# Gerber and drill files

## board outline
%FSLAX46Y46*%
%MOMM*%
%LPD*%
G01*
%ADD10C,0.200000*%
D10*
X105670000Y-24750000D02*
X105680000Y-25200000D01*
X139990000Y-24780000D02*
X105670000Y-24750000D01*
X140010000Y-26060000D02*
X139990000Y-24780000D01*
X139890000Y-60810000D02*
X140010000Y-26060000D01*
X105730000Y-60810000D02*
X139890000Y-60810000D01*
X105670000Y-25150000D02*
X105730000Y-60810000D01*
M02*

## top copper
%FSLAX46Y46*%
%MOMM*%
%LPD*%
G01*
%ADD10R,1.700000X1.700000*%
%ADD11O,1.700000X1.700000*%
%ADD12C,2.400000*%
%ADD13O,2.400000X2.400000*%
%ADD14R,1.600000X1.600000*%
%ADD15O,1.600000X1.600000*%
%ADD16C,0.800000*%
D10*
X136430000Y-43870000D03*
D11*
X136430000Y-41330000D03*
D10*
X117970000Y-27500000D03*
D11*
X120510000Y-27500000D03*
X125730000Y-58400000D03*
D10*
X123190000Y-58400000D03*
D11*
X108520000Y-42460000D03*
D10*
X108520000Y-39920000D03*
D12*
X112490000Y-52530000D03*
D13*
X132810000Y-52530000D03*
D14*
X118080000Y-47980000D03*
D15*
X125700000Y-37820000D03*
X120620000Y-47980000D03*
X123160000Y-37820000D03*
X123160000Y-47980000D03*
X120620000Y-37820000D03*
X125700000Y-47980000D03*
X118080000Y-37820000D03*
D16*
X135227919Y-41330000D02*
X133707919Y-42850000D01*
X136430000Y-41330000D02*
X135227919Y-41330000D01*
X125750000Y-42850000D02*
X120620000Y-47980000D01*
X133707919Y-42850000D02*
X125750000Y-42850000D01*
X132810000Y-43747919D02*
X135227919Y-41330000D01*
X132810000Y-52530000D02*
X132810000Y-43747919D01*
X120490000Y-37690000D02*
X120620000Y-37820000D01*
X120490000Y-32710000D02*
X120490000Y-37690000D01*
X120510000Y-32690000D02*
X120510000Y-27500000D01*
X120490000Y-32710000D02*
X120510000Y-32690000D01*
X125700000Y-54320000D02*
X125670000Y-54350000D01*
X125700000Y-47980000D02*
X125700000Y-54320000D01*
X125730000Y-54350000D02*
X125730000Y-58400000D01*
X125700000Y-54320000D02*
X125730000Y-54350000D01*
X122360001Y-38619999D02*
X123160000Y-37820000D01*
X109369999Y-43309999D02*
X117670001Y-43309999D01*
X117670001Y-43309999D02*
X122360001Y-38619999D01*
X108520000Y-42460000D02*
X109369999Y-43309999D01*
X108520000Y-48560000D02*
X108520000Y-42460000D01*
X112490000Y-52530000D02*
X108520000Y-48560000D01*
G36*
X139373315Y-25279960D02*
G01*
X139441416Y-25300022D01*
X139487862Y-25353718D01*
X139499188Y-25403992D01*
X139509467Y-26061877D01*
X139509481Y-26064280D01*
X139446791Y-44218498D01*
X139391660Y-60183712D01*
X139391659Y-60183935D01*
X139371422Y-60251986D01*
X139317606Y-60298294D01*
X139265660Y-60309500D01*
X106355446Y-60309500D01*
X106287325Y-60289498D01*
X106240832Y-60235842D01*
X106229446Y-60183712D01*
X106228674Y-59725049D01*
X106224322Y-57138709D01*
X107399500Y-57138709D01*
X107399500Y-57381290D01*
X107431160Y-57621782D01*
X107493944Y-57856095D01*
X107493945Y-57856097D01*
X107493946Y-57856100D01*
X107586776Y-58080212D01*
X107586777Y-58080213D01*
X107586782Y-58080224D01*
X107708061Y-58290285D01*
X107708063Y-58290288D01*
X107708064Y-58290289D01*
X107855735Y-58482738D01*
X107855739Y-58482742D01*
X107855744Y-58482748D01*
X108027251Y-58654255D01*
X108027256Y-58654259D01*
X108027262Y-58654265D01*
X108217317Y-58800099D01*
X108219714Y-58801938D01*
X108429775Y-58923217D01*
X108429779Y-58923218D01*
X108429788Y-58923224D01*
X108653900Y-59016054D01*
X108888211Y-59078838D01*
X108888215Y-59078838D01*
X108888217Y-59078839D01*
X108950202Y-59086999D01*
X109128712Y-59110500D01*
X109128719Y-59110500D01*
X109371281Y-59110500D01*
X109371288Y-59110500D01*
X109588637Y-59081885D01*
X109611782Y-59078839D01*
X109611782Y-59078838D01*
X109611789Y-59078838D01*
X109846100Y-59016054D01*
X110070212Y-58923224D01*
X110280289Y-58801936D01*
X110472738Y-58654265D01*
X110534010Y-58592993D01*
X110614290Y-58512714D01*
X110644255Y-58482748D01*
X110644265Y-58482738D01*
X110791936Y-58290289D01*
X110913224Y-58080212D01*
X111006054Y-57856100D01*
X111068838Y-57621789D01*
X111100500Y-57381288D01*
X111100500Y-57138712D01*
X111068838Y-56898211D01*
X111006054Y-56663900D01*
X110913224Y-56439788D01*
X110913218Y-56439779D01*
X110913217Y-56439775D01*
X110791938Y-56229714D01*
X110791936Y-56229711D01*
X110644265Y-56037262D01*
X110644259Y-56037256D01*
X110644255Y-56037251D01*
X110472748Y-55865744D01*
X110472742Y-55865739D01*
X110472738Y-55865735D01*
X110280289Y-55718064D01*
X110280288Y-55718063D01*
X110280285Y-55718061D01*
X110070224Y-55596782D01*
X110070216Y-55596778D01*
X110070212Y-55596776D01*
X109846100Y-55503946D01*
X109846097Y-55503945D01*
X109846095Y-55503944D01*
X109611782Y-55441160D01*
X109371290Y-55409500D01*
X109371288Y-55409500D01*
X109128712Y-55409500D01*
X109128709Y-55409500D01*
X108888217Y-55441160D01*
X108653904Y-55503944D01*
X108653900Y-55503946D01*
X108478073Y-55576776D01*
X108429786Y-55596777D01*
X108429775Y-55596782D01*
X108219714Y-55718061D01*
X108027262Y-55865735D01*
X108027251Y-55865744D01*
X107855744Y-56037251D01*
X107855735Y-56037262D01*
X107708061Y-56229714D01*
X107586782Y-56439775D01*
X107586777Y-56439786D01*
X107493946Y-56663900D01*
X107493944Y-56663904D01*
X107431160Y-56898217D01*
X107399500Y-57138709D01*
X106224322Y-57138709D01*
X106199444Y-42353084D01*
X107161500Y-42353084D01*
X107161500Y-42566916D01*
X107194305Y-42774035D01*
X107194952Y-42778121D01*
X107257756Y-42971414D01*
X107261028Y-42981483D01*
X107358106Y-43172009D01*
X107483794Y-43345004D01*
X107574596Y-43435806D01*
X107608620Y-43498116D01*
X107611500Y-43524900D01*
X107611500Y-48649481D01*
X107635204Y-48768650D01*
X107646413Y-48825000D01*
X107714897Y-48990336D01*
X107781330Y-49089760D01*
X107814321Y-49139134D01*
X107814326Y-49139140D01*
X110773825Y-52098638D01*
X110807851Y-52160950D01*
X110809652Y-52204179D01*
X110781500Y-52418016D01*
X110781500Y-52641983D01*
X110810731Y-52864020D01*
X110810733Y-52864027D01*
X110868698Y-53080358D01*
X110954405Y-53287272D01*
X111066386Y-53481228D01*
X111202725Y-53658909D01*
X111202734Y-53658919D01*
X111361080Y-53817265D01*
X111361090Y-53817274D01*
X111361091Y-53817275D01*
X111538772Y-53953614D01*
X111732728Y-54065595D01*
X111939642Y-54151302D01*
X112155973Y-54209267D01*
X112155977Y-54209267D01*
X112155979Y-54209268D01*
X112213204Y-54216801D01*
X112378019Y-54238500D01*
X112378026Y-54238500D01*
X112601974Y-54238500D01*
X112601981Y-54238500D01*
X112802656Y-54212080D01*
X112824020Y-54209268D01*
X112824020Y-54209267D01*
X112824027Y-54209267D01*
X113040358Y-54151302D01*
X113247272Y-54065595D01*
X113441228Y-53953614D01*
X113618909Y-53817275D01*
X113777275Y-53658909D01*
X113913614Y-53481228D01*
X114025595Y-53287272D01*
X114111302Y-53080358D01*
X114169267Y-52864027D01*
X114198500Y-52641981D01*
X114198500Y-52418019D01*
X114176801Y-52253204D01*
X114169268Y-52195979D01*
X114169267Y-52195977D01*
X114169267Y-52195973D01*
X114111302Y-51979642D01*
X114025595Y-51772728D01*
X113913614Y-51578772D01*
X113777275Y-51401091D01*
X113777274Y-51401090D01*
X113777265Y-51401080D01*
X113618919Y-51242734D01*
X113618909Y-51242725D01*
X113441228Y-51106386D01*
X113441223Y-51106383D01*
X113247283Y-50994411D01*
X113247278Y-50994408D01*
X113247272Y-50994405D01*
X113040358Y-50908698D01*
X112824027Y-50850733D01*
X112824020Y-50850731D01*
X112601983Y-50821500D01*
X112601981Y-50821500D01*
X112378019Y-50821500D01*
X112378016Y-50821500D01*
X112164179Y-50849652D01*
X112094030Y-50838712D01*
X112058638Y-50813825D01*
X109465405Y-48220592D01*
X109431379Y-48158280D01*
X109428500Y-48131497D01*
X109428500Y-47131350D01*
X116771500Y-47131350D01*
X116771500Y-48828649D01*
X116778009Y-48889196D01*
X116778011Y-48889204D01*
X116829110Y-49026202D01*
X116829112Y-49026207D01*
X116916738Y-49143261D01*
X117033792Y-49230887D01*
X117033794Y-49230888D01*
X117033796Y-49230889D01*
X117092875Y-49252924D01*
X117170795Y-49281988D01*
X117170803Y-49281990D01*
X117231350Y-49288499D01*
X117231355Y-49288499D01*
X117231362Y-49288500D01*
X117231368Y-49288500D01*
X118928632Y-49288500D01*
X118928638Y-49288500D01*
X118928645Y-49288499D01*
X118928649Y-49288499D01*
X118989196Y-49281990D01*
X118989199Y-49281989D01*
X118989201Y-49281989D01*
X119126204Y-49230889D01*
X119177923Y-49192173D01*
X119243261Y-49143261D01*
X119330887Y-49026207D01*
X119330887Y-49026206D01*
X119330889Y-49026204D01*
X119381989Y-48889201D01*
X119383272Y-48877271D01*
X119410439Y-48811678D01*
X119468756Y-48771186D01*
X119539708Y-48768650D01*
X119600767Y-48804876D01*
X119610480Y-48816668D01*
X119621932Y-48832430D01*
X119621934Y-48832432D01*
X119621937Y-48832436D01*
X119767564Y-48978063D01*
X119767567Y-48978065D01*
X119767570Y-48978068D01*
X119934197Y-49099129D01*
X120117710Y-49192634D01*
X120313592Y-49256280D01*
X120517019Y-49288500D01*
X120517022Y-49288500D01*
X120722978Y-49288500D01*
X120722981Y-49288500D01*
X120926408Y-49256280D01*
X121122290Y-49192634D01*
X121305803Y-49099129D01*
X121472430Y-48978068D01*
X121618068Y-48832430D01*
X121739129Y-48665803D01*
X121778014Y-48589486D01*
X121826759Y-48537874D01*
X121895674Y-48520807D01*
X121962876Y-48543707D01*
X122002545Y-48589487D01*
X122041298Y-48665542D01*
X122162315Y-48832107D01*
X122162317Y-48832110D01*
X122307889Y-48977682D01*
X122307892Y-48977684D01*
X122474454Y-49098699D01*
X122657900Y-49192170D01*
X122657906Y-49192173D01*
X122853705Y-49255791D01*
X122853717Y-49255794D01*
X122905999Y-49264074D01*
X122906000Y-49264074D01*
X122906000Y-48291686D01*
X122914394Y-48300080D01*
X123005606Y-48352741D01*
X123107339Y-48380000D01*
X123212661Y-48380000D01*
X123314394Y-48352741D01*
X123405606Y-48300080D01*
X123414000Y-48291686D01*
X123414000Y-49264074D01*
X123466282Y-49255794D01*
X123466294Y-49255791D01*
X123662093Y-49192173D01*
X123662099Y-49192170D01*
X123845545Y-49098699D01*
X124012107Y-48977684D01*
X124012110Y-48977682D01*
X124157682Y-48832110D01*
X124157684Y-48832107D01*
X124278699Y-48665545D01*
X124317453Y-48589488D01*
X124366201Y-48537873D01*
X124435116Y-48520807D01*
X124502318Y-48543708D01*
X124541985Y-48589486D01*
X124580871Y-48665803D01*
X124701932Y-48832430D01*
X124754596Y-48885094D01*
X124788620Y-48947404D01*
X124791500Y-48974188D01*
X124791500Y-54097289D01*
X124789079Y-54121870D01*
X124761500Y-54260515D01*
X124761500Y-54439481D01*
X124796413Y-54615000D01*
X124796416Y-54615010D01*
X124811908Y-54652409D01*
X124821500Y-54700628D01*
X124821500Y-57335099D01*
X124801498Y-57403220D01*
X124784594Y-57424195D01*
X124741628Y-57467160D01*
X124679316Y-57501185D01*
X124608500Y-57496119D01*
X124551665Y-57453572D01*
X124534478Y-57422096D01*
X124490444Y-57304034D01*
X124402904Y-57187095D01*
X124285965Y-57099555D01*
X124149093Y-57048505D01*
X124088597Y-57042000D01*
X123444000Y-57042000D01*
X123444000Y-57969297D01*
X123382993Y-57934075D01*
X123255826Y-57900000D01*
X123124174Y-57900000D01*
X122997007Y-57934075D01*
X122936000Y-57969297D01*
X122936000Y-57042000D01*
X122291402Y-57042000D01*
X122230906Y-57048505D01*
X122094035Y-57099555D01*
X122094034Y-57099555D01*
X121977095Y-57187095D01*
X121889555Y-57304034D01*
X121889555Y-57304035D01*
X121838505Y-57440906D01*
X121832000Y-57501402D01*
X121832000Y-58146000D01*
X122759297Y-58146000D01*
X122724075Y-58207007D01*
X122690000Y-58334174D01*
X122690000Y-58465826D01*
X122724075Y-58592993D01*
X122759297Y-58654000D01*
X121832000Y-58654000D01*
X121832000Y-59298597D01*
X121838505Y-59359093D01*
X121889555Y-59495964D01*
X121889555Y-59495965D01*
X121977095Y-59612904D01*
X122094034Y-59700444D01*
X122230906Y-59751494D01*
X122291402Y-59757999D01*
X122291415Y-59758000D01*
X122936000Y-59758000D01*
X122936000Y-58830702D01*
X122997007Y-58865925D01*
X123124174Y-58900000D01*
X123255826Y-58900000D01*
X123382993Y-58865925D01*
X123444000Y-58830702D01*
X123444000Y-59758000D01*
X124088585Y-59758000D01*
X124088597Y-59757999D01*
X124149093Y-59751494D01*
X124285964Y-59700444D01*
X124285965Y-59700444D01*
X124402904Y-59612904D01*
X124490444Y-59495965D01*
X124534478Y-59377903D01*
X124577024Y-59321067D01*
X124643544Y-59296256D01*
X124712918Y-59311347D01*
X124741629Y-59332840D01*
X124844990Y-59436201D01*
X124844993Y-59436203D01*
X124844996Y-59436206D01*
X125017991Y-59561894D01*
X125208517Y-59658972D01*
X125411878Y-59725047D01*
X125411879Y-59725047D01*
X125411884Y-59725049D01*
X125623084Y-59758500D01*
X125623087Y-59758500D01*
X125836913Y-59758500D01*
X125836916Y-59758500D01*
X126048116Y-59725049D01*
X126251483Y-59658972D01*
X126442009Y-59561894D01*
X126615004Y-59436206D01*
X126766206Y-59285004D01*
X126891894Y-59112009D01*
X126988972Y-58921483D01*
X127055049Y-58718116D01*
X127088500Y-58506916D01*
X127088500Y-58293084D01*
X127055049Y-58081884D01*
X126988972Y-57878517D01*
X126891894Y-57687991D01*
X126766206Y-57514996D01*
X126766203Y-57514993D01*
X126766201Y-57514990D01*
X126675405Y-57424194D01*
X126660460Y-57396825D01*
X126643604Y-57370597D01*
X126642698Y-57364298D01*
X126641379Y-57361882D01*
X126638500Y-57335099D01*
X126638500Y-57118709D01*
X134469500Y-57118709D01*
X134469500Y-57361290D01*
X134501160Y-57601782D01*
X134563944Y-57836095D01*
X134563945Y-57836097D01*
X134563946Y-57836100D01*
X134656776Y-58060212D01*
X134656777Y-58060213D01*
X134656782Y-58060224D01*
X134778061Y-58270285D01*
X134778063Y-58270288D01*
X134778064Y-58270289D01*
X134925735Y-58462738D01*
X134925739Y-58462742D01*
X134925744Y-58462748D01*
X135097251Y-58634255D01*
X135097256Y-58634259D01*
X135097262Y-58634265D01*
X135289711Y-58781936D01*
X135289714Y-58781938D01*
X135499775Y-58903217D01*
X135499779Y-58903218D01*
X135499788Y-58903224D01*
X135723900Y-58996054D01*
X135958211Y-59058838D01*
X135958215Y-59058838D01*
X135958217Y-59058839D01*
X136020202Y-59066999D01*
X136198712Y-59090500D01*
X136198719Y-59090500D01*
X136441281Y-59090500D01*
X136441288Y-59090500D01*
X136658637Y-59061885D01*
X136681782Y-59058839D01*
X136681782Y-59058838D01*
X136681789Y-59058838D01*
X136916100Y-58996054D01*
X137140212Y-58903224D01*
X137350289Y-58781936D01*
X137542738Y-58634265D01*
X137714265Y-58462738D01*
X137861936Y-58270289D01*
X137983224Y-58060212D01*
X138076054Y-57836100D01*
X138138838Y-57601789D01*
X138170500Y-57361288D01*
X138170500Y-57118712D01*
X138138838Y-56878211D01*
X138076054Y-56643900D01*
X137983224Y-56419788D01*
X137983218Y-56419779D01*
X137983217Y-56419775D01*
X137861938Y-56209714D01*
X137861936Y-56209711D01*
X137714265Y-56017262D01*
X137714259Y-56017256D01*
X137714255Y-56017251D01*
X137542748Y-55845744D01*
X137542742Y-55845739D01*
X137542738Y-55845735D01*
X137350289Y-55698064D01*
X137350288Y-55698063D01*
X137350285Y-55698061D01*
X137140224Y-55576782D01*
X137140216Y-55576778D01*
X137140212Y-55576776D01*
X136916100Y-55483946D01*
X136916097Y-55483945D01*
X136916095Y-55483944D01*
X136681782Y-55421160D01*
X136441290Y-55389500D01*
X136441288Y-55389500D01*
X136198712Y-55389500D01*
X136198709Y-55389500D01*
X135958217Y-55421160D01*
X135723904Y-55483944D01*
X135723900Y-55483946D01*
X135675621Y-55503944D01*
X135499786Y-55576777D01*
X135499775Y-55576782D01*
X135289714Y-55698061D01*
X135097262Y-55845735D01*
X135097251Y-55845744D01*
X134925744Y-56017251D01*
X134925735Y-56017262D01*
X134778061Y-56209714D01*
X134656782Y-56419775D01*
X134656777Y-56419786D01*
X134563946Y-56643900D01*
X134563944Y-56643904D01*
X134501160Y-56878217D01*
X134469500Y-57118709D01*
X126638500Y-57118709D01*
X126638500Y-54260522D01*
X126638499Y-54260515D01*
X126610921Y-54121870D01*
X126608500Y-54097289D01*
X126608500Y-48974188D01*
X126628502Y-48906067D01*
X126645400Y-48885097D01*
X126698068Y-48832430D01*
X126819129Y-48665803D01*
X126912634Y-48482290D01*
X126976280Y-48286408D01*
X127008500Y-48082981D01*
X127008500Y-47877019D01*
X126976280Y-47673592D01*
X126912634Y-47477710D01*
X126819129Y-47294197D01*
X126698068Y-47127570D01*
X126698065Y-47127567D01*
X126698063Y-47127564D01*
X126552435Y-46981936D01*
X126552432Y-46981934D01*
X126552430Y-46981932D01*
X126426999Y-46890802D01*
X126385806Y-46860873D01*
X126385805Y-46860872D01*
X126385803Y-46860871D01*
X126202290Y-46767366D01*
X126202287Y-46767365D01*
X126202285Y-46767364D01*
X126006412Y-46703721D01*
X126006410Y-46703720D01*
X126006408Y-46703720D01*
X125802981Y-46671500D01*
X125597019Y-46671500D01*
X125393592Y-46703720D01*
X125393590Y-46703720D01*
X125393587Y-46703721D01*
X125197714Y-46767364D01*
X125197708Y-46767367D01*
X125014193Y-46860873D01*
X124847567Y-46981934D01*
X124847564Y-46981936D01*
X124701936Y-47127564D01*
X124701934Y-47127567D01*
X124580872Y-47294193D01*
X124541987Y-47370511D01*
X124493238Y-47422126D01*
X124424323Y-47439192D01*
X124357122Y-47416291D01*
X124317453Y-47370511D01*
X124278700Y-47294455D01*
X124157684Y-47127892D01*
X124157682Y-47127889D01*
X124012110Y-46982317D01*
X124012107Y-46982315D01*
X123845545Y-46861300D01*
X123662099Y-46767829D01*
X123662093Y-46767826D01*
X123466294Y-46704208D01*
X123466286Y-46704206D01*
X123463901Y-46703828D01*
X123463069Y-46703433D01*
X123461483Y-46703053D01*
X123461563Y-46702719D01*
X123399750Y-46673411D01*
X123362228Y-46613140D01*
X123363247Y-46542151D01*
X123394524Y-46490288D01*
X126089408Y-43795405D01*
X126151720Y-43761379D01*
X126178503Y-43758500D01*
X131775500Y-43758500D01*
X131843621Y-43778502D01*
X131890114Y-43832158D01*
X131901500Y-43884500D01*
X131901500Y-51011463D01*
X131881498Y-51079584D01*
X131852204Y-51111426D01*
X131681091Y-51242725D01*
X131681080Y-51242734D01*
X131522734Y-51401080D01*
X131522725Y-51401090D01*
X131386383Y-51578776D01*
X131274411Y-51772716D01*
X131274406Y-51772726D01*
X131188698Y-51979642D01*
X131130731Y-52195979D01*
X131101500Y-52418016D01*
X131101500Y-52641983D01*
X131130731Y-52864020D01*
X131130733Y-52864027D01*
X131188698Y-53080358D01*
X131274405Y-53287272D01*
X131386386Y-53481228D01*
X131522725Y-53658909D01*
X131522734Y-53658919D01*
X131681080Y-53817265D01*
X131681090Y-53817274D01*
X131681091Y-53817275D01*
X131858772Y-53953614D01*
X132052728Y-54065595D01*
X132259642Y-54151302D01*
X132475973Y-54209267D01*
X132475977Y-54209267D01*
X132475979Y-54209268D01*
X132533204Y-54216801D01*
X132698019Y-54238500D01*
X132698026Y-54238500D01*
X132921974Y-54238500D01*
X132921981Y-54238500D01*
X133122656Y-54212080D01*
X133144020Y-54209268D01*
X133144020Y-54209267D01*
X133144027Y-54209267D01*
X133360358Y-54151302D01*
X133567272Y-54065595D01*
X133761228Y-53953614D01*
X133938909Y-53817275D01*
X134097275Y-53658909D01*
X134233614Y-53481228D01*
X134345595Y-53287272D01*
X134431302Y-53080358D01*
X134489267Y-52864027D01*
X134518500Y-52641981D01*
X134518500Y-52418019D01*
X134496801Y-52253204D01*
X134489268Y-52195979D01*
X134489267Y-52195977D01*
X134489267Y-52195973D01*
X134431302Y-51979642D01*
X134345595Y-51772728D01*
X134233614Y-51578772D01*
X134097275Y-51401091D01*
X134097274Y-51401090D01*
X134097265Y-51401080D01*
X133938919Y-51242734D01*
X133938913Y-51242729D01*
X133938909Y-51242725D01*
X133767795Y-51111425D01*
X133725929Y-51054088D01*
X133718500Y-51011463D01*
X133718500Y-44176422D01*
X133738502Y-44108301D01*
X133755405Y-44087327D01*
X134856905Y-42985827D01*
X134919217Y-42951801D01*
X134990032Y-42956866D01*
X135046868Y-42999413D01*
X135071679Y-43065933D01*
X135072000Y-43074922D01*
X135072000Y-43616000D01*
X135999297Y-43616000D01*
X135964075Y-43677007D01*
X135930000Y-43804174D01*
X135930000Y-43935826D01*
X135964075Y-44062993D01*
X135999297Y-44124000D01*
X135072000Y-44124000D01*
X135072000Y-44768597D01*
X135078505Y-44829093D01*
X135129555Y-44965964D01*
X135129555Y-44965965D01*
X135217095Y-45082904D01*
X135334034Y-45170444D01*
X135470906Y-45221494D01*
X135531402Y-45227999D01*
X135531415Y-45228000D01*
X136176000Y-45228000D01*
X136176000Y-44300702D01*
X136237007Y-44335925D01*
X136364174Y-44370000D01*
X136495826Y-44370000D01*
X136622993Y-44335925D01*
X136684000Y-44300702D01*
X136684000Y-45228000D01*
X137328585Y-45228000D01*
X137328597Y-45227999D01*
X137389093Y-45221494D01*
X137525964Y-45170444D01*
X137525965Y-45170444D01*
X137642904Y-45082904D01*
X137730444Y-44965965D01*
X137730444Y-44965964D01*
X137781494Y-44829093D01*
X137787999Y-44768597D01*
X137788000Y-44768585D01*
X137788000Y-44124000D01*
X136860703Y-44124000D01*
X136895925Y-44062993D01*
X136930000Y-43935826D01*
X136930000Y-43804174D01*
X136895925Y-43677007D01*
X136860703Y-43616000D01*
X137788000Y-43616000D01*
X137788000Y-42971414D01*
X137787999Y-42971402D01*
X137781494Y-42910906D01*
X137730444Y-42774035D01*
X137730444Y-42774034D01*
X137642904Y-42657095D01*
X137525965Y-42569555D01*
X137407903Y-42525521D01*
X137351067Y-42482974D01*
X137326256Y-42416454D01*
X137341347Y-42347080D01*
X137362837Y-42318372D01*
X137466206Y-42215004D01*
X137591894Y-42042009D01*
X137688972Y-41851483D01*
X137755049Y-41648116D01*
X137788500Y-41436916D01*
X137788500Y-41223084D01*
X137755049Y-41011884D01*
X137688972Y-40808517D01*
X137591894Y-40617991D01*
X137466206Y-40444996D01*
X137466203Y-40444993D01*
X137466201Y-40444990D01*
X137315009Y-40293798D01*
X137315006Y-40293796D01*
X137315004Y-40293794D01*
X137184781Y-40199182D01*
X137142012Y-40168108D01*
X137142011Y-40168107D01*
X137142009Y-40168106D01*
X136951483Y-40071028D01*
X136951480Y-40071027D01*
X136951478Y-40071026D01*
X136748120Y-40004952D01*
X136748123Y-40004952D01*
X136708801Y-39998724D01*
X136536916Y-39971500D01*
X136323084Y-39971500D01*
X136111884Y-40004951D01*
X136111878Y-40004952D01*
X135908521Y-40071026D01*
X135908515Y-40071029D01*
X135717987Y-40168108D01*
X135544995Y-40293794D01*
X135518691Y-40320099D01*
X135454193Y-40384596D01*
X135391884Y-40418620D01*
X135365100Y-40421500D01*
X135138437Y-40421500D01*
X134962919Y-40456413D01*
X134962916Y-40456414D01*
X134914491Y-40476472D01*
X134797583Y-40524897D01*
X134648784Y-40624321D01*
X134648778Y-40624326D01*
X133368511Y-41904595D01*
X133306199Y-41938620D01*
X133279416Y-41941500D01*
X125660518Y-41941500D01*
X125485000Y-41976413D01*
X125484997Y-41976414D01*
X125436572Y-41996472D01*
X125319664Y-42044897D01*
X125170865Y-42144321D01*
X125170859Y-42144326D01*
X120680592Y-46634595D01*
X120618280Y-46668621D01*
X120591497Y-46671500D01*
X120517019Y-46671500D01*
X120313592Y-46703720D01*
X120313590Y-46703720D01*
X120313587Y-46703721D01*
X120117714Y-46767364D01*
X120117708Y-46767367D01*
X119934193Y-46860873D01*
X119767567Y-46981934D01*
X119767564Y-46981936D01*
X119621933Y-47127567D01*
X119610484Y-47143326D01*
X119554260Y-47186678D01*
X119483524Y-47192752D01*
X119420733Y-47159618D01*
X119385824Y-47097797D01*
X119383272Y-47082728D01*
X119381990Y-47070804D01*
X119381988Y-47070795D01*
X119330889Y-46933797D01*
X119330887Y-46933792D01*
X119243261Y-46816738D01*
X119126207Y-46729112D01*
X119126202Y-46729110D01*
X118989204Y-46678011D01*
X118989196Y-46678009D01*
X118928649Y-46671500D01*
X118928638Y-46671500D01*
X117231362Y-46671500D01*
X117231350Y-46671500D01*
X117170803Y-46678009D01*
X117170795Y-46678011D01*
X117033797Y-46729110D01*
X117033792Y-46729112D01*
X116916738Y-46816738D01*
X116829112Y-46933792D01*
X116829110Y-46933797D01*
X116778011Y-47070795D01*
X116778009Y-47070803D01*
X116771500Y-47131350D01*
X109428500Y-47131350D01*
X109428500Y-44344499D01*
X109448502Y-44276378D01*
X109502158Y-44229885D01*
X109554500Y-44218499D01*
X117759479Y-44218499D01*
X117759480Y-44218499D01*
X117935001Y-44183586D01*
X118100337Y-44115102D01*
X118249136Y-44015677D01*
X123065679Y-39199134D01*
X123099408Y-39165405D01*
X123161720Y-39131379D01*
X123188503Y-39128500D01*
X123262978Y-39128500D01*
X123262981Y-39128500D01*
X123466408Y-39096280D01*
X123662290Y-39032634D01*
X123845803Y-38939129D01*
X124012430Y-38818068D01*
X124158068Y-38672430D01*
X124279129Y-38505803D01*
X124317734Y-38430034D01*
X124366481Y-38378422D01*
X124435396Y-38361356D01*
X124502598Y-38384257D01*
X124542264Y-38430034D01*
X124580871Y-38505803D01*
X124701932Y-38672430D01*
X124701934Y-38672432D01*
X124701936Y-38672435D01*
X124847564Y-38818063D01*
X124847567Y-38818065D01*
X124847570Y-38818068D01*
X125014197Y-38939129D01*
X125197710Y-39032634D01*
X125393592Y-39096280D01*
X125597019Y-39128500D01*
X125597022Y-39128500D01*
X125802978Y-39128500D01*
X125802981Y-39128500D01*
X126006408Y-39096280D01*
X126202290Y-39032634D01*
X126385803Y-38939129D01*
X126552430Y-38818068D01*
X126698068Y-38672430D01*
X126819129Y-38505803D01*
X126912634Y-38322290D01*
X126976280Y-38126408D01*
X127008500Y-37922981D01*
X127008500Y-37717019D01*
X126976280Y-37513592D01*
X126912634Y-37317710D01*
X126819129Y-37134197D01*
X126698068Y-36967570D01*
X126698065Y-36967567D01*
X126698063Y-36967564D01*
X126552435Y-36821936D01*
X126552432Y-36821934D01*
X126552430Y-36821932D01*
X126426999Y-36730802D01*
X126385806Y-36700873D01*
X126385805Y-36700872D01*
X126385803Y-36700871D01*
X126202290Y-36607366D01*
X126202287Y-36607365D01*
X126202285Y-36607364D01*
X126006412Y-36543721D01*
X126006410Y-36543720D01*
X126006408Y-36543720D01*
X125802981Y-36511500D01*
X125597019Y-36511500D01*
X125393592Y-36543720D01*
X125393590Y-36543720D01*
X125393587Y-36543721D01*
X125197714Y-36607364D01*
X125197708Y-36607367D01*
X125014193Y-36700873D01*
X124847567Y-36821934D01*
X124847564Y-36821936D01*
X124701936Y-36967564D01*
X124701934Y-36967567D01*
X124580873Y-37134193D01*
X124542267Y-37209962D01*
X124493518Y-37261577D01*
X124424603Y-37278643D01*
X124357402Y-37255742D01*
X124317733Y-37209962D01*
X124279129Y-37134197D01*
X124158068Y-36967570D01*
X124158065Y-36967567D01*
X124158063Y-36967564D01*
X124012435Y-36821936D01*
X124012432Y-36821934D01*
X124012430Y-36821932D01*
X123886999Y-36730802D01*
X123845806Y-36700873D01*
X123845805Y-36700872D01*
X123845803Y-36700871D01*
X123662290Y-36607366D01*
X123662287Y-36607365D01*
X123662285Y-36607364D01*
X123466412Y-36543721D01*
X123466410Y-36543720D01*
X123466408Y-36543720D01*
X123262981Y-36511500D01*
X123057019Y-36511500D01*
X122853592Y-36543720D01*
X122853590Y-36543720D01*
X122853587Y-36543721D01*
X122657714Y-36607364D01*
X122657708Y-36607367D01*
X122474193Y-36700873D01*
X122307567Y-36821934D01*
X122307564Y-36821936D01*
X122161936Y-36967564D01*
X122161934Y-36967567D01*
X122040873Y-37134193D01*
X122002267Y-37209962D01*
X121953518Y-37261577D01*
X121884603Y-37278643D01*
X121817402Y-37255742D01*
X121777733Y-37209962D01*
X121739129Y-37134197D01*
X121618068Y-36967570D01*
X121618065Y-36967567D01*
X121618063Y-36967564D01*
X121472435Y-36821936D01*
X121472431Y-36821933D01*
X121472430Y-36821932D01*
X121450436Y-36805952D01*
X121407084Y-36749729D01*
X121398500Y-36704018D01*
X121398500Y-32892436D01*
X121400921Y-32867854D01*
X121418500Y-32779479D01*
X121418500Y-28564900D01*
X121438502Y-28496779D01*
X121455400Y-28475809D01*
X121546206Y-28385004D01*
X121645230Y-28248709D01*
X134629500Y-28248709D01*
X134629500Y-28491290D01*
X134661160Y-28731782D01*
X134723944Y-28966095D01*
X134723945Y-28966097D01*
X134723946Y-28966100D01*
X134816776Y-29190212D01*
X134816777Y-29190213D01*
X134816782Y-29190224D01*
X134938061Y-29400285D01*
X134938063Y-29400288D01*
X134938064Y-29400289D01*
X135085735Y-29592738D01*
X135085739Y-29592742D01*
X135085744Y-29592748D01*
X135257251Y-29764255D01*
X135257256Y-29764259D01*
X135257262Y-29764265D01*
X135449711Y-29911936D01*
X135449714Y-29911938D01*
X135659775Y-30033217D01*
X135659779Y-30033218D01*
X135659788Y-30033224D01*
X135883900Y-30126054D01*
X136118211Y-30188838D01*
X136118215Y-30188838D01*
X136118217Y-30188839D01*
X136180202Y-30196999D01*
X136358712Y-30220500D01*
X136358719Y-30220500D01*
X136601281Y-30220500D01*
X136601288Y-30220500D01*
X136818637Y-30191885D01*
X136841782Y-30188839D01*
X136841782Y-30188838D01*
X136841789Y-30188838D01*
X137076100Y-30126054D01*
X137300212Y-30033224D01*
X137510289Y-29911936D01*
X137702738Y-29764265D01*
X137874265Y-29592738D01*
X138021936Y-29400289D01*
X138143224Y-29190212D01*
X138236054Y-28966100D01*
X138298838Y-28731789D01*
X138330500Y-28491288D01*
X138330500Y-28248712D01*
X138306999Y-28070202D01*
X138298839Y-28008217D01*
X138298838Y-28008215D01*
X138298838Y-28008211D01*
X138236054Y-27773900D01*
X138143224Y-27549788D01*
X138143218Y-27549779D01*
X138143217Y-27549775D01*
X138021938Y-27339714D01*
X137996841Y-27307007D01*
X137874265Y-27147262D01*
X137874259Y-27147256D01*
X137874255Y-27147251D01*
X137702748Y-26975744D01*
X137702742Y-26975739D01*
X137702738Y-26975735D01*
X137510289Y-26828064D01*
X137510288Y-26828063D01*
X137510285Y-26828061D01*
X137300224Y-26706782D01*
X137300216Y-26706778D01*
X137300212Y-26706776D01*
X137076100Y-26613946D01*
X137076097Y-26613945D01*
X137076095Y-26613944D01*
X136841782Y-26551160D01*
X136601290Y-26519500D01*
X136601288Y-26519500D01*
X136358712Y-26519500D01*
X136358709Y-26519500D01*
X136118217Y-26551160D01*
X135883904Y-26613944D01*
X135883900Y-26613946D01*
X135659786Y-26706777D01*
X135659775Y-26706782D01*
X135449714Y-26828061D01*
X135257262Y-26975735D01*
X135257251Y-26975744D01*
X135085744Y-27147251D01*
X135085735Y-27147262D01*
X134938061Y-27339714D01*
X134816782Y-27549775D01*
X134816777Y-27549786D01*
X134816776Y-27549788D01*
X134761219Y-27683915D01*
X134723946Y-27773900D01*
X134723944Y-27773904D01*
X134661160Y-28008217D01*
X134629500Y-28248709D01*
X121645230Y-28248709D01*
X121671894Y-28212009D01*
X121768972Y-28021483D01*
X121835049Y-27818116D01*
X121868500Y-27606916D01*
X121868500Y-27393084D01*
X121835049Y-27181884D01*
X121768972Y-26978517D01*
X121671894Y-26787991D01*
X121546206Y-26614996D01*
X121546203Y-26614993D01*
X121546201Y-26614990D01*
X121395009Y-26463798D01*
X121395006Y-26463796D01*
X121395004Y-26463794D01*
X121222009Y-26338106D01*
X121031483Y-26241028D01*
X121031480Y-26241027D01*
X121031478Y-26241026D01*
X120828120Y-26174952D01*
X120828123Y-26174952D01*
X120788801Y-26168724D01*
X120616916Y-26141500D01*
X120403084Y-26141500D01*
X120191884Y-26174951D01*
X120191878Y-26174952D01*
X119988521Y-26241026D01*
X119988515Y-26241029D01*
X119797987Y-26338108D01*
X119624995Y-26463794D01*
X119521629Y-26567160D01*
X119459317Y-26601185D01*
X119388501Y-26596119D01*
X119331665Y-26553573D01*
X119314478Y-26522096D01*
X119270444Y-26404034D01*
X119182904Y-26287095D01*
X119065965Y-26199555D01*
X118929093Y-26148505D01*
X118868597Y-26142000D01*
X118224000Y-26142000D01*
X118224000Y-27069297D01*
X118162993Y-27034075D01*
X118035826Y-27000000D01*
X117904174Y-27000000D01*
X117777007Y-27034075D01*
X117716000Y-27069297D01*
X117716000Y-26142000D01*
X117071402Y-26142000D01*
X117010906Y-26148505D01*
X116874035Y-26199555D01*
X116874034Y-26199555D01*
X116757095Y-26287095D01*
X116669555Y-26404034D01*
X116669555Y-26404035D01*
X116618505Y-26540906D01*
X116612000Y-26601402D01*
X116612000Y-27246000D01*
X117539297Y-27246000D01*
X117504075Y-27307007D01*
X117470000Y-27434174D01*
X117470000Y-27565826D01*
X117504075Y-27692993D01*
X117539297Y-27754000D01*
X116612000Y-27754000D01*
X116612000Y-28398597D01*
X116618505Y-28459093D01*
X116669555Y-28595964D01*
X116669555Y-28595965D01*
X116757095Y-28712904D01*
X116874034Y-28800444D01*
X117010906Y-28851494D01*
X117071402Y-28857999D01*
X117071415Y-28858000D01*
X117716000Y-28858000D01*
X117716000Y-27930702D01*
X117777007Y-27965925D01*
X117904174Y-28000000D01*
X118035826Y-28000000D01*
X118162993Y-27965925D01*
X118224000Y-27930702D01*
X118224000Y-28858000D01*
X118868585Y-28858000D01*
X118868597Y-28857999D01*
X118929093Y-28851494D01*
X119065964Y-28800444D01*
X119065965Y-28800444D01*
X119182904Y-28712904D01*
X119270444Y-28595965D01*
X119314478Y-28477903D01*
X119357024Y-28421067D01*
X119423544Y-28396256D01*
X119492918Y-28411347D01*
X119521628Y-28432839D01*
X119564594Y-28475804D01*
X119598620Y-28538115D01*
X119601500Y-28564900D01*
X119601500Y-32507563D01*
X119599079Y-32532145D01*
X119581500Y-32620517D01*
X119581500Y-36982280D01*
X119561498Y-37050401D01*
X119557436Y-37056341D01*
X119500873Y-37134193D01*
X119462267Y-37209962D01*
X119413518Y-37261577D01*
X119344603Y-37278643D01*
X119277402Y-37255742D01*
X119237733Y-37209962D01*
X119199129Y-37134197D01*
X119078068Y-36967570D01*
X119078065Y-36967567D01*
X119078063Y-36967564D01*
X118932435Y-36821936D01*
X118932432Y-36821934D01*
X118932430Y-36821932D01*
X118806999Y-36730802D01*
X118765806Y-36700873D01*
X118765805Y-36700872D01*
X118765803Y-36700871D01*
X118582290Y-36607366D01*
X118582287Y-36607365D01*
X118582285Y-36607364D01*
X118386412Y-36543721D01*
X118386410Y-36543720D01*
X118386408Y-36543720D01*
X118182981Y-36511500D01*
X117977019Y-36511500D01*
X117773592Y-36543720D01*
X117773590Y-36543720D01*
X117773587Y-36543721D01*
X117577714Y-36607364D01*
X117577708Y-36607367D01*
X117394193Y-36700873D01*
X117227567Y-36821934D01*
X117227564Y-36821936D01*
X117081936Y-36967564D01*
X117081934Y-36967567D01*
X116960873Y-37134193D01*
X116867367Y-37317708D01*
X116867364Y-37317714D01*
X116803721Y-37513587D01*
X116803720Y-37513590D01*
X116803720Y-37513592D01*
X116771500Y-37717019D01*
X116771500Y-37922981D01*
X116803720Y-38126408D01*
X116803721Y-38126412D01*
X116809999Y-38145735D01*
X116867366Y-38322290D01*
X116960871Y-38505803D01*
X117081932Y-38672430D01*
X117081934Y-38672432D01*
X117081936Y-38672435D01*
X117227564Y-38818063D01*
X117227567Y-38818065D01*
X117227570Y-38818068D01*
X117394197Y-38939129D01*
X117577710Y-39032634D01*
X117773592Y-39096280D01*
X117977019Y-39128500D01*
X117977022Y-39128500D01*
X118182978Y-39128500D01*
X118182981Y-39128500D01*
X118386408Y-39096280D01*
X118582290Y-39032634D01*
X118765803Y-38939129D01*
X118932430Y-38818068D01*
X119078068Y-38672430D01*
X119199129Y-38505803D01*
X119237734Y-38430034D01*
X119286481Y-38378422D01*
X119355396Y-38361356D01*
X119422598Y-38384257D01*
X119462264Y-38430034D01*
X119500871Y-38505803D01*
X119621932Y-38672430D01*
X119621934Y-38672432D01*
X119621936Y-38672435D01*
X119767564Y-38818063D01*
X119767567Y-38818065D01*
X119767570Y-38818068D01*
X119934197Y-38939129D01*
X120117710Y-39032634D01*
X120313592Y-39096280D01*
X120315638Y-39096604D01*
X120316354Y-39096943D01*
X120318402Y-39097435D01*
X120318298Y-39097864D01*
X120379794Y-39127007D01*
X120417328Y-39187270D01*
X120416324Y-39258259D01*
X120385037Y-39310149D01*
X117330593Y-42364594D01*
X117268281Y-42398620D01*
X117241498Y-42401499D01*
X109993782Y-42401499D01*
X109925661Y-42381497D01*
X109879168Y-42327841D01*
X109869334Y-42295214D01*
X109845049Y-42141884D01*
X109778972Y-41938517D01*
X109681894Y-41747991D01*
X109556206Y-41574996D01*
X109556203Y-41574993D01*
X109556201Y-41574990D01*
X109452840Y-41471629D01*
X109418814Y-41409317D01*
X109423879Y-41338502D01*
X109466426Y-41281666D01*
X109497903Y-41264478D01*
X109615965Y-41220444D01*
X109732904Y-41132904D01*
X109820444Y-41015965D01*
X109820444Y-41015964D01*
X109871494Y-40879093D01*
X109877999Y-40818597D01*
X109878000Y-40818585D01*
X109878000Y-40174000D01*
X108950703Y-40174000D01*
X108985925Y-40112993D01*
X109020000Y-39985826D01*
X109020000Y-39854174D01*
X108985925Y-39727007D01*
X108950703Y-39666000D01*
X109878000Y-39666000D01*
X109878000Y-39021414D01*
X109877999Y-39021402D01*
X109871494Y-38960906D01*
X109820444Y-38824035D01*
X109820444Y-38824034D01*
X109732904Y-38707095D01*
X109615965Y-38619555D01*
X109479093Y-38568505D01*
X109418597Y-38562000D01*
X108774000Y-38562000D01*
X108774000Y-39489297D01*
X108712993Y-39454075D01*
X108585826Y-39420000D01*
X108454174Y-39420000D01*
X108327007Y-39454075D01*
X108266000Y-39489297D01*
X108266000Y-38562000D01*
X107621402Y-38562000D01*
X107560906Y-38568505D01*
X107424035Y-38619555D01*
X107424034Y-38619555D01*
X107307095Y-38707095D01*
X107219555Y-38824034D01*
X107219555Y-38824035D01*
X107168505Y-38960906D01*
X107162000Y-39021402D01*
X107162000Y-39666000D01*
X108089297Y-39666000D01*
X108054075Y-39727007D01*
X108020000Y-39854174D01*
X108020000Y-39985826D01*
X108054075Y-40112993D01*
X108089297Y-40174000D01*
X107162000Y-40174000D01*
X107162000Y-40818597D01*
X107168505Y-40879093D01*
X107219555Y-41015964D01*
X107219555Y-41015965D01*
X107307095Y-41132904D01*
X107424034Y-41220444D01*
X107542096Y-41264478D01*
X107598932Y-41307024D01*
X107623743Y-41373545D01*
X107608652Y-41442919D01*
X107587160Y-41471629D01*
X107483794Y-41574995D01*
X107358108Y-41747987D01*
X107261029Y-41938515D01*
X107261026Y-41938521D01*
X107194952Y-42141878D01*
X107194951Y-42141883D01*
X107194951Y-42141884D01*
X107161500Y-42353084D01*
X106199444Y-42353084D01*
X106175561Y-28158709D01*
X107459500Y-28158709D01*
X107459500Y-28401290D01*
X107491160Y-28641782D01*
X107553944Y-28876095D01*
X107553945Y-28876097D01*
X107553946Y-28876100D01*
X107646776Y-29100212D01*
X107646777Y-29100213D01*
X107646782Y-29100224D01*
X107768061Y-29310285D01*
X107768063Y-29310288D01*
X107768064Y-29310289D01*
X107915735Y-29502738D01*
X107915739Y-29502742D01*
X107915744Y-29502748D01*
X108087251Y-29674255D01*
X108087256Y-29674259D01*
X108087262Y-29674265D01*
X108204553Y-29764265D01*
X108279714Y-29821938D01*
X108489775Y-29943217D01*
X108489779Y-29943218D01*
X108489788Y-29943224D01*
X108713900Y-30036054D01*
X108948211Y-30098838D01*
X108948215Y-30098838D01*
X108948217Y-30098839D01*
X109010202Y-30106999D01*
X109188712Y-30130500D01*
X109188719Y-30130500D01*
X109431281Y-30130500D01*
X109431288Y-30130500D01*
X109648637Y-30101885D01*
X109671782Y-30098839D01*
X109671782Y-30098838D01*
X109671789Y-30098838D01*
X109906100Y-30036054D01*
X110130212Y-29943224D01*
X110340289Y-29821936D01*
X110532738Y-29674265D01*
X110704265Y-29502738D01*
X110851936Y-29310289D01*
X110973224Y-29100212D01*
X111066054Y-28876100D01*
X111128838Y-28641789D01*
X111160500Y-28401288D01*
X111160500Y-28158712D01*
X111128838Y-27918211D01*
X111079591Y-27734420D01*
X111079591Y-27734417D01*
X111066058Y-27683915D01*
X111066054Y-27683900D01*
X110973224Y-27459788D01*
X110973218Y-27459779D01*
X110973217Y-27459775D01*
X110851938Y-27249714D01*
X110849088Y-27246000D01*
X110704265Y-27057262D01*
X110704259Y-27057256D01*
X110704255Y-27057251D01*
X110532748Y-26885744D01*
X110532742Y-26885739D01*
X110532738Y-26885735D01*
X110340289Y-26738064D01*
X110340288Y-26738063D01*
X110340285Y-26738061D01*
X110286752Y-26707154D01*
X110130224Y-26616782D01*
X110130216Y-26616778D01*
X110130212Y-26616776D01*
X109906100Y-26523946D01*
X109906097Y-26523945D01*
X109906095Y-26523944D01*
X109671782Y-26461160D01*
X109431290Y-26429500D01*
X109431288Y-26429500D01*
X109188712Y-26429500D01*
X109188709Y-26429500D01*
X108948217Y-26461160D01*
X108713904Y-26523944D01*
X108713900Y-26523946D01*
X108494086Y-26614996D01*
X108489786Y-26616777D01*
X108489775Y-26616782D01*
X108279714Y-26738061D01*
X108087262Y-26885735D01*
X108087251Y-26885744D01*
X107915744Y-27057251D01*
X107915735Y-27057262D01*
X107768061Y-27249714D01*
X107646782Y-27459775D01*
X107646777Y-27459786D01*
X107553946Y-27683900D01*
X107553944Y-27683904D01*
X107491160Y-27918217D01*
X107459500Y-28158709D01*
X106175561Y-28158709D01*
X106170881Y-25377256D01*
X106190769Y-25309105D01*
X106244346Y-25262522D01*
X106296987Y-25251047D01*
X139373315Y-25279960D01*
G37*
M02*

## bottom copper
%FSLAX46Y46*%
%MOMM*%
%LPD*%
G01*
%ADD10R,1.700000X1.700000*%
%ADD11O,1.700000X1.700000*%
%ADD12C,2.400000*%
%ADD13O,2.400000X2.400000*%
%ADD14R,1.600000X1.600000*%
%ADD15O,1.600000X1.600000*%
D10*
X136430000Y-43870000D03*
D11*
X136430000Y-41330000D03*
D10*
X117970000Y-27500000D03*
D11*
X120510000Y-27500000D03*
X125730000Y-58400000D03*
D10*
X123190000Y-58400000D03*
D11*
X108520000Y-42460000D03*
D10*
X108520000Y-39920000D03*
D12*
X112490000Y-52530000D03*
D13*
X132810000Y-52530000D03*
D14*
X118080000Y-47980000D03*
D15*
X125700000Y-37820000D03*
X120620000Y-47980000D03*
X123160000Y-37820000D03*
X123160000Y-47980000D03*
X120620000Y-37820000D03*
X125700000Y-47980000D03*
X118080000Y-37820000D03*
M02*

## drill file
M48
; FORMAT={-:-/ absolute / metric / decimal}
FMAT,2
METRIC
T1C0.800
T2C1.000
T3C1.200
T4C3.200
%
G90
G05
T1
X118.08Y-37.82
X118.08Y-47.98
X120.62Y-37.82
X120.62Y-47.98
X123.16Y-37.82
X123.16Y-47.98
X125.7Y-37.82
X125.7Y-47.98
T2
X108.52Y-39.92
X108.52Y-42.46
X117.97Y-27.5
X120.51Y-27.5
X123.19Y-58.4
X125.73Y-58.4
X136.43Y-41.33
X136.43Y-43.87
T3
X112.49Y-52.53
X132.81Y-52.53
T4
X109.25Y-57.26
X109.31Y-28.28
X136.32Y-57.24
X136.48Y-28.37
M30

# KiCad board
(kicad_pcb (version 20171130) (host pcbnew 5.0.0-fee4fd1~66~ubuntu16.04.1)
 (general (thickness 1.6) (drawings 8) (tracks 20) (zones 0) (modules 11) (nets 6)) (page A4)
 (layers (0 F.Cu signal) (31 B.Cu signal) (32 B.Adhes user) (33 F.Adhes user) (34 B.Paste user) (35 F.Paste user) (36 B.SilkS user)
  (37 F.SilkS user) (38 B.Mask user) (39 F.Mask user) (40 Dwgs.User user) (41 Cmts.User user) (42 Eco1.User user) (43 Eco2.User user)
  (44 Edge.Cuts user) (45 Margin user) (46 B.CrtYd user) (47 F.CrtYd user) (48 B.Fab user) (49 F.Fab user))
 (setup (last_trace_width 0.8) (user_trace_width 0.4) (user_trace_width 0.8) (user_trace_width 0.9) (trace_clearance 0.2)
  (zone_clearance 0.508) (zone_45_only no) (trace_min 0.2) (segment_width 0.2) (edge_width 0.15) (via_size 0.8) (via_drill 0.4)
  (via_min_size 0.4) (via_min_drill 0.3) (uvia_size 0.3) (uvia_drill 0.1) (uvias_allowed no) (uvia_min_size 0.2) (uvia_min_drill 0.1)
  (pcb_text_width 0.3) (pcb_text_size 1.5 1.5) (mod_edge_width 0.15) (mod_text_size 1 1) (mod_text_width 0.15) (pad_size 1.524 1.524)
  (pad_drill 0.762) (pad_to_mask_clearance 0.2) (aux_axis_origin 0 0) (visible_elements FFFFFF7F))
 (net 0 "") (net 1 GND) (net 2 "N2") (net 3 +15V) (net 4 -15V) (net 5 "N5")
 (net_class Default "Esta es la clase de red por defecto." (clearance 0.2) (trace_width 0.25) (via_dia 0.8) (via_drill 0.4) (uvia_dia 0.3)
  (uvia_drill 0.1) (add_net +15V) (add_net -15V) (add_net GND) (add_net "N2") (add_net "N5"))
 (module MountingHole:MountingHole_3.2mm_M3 (layer F.Cu) (at 136.32 57.24)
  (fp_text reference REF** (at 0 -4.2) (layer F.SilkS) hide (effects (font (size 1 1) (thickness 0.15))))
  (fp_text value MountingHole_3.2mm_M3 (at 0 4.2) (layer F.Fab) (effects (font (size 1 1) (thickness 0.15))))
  (pad 1 np_thru_hole circle (at 0 0) (size 3.2 3.2) (drill 3.2) (layers *.Cu *.Mask)))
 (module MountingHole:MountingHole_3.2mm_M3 (layer F.Cu) (at 109.25 57.26)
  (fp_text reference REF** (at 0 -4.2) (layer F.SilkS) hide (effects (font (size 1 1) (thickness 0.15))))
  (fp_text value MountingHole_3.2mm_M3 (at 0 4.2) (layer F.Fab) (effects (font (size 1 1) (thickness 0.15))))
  (pad 1 np_thru_hole circle (at 0 0) (size 3.2 3.2) (drill 3.2) (layers *.Cu *.Mask)))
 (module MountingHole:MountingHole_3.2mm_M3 (layer F.Cu) (at 109.31 28.28)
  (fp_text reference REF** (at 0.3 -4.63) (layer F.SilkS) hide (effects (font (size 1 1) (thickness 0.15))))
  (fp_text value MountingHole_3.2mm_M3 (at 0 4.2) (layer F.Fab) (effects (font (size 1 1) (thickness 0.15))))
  (pad 1 np_thru_hole circle (at 0 0) (size 3.2 3.2) (drill 3.2) (layers *.Cu *.Mask)))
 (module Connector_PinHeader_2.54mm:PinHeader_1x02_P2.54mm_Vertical (layer F.Cu) (at 136.43 43.87 180)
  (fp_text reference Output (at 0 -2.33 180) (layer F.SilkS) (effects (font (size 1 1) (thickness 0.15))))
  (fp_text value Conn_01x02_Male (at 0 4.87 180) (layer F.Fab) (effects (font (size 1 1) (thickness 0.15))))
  (pad 1 thru_hole rect (at 0 0 180) (size 1.7 1.7) (drill 1) (layers *.Cu *.Mask) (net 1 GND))
  (pad 2 thru_hole oval (at 0 2.54 180) (size 1.7 1.7) (drill 1) (layers *.Cu *.Mask) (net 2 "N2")))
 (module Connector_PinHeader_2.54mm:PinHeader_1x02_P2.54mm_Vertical (layer F.Cu) (at 117.97 27.5 90)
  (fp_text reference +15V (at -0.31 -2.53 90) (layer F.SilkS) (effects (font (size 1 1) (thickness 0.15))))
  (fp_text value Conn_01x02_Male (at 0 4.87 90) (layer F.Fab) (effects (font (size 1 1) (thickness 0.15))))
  (pad 1 thru_hole rect (at 0 0 90) (size 1.7 1.7) (drill 1) (layers *.Cu *.Mask) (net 1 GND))
  (pad 2 thru_hole oval (at 0 2.54 90) (size 1.7 1.7) (drill 1) (layers *.Cu *.Mask) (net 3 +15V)))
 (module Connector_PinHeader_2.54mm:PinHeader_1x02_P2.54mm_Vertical (layer F.Cu) (at 123.19 58.4 90)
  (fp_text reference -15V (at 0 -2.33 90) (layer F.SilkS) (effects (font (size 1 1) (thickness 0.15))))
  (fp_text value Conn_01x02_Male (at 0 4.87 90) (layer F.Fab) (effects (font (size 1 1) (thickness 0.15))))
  (pad 2 thru_hole oval (at 0 2.54 90) (size 1.7 1.7) (drill 1) (layers *.Cu *.Mask) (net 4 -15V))
  (pad 1 thru_hole rect (at 0 0 90) (size 1.7 1.7) (drill 1) (layers *.Cu *.Mask) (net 1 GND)))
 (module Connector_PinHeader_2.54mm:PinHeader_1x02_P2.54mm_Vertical (layer F.Cu) (at 108.52 39.92)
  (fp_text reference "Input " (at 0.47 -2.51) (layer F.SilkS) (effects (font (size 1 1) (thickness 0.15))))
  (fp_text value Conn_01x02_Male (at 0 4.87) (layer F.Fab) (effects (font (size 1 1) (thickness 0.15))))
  (pad 2 thru_hole oval (at 0 2.54) (size 1.7 1.7) (drill 1) (layers *.Cu *.Mask) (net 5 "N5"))
  (pad 1 thru_hole rect (at 0 0) (size 1.7 1.7) (drill 1) (layers *.Cu *.Mask) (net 1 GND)))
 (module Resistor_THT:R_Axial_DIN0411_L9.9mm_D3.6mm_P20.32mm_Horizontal (layer F.Cu) (at 112.49 52.53)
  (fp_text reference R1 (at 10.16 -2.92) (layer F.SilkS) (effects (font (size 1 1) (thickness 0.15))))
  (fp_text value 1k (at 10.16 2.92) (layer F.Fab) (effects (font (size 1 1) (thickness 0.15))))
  (pad 1 thru_hole circle (at 0 0) (size 2.4 2.4) (drill 1.2) (layers *.Cu *.Mask) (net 5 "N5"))
  (pad 2 thru_hole oval (at 20.32 0) (size 2.4 2.4) (drill 1.2) (layers *.Cu *.Mask) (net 2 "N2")))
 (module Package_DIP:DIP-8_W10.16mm (layer F.Cu) (at 118.08 47.98 90)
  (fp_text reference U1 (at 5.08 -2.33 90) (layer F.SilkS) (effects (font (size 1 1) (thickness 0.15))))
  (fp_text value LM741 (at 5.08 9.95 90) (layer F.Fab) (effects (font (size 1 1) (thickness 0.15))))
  (pad 1 thru_hole rect (at 0 0 90) (size 1.6 1.6) (drill 0.8) (layers *.Cu *.Mask))
  (pad 5 thru_hole oval (at 10.16 7.62 90) (size 1.6 1.6) (drill 0.8) (layers *.Cu *.Mask))
  (pad 2 thru_hole oval (at 0 2.54 90) (size 1.6 1.6) (drill 0.8) (layers *.Cu *.Mask) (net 2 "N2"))
  (pad 6 thru_hole oval (at 10.16 5.08 90) (size 1.6 1.6) (drill 0.8) (layers *.Cu *.Mask) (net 5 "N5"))
  (pad 3 thru_hole oval (at 0 5.08 90) (size 1.6 1.6) (drill 0.8) (layers *.Cu *.Mask) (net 1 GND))
  (pad 7 thru_hole oval (at 10.16 2.54 90) (size 1.6 1.6) (drill 0.8) (layers *.Cu *.Mask) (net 3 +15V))
  (pad 4 thru_hole oval (at 0 7.62 90) (size 1.6 1.6) (drill 0.8) (layers *.Cu *.Mask) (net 4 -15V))
  (pad 8 thru_hole oval (at 10.16 0 90) (size 1.6 1.6) (drill 0.8) (layers *.Cu *.Mask)))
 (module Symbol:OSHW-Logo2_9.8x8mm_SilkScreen (layer F.Cu) (at 127.92 30.9 90)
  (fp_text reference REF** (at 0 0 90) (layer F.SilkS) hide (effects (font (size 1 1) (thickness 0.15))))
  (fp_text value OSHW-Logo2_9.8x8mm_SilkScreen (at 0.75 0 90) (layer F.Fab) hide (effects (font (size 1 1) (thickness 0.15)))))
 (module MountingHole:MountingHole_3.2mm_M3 (layer F.Cu) (at 136.48 28.37)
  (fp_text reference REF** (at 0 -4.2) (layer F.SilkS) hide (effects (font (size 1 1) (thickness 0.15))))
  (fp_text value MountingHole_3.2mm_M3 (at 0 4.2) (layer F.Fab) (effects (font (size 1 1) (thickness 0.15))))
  (pad 1 np_thru_hole circle (at 0 0) (size 3.2 3.2) (drill 3.2) (layers *.Cu *.Mask)))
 (gr_line (start 105.67 24.75) (end 105.68 25.2) (layer Edge.Cuts) (width 0.2))
 (gr_line (start 139.99 24.78) (end 105.67 24.75) (layer Edge.Cuts) (width 0.2))
 (gr_line (start 140.01 26.06) (end 139.99 24.78) (layer Edge.Cuts) (width 0.2))
 (gr_line (start 139.89 60.81) (end 140.01 26.06) (layer Edge.Cuts) (width 0.2))
 (gr_line (start 105.73 60.81) (end 139.89 60.81) (layer Edge.Cuts) (width 0.2))
 (gr_line (start 105.67 25.15) (end 105.73 60.81) (layer Edge.Cuts) (width 0.2))
 (segment (start 135.227919 41.33) (end 133.707919 42.85) (width 0.8) (layer F.Cu) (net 2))
 (segment (start 136.43 41.33) (end 135.227919 41.33) (width 0.8) (layer F.Cu) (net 2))
 (segment (start 125.75 42.85) (end 120.62 47.98) (width 0.8) (layer F.Cu) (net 2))
 (segment (start 133.707919 42.85) (end 125.75 42.85) (width 0.8) (layer F.Cu) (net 2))
 (segment (start 132.81 43.747919) (end 135.227919 41.33) (width 0.8) (layer F.Cu) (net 2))
 (segment (start 132.81 52.53) (end 132.81 43.747919) (width 0.8) (layer F.Cu) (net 2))
 (segment (start 120.49 37.69) (end 120.62 37.82) (width 0.8) (layer F.Cu) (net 3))
 (segment (start 120.49 32.71) (end 120.49 37.69) (width 0.8) (layer F.Cu) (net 3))
 (segment (start 120.51 32.69) (end 120.51 27.5) (width 0.8) (layer F.Cu) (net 3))
 (segment (start 120.49 32.71) (end 120.51 32.69) (width 0.8) (layer F.Cu) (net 3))
 (segment (start 125.7 54.32) (end 125.67 54.35) (width 0.8) (layer F.Cu) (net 4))
 (segment (start 125.7 47.98) (end 125.7 54.32) (width 0.8) (layer F.Cu) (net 4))
 (segment (start 125.73 54.35) (end 125.73 58.4) (width 0.8) (layer F.Cu) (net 4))
 (segment (start 125.7 54.32) (end 125.73 54.35) (width 0.8) (layer F.Cu) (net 4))
 (segment (start 122.360001 38.619999) (end 123.16 37.82) (width 0.8) (layer F.Cu) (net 5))
 (segment (start 109.369999 43.309999) (end 117.670001 43.309999) (width 0.8) (layer F.Cu) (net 5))
 (segment (start 117.670001 43.309999) (end 122.360001 38.619999) (width 0.8) (layer F.Cu) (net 5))
 (segment (start 108.52 42.46) (end 109.369999 43.309999) (width 0.8) (layer F.Cu) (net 5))
 (segment (start 108.52 48.56) (end 108.52 42.46) (width 0.8) (layer F.Cu) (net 5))
 (segment (start 112.49 52.53) (end 108.52 48.56) (width 0.8) (layer F.Cu) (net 5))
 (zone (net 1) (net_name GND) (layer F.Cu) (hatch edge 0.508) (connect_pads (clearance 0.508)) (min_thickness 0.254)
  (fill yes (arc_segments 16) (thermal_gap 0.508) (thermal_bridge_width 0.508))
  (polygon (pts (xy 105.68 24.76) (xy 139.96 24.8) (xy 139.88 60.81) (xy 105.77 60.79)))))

